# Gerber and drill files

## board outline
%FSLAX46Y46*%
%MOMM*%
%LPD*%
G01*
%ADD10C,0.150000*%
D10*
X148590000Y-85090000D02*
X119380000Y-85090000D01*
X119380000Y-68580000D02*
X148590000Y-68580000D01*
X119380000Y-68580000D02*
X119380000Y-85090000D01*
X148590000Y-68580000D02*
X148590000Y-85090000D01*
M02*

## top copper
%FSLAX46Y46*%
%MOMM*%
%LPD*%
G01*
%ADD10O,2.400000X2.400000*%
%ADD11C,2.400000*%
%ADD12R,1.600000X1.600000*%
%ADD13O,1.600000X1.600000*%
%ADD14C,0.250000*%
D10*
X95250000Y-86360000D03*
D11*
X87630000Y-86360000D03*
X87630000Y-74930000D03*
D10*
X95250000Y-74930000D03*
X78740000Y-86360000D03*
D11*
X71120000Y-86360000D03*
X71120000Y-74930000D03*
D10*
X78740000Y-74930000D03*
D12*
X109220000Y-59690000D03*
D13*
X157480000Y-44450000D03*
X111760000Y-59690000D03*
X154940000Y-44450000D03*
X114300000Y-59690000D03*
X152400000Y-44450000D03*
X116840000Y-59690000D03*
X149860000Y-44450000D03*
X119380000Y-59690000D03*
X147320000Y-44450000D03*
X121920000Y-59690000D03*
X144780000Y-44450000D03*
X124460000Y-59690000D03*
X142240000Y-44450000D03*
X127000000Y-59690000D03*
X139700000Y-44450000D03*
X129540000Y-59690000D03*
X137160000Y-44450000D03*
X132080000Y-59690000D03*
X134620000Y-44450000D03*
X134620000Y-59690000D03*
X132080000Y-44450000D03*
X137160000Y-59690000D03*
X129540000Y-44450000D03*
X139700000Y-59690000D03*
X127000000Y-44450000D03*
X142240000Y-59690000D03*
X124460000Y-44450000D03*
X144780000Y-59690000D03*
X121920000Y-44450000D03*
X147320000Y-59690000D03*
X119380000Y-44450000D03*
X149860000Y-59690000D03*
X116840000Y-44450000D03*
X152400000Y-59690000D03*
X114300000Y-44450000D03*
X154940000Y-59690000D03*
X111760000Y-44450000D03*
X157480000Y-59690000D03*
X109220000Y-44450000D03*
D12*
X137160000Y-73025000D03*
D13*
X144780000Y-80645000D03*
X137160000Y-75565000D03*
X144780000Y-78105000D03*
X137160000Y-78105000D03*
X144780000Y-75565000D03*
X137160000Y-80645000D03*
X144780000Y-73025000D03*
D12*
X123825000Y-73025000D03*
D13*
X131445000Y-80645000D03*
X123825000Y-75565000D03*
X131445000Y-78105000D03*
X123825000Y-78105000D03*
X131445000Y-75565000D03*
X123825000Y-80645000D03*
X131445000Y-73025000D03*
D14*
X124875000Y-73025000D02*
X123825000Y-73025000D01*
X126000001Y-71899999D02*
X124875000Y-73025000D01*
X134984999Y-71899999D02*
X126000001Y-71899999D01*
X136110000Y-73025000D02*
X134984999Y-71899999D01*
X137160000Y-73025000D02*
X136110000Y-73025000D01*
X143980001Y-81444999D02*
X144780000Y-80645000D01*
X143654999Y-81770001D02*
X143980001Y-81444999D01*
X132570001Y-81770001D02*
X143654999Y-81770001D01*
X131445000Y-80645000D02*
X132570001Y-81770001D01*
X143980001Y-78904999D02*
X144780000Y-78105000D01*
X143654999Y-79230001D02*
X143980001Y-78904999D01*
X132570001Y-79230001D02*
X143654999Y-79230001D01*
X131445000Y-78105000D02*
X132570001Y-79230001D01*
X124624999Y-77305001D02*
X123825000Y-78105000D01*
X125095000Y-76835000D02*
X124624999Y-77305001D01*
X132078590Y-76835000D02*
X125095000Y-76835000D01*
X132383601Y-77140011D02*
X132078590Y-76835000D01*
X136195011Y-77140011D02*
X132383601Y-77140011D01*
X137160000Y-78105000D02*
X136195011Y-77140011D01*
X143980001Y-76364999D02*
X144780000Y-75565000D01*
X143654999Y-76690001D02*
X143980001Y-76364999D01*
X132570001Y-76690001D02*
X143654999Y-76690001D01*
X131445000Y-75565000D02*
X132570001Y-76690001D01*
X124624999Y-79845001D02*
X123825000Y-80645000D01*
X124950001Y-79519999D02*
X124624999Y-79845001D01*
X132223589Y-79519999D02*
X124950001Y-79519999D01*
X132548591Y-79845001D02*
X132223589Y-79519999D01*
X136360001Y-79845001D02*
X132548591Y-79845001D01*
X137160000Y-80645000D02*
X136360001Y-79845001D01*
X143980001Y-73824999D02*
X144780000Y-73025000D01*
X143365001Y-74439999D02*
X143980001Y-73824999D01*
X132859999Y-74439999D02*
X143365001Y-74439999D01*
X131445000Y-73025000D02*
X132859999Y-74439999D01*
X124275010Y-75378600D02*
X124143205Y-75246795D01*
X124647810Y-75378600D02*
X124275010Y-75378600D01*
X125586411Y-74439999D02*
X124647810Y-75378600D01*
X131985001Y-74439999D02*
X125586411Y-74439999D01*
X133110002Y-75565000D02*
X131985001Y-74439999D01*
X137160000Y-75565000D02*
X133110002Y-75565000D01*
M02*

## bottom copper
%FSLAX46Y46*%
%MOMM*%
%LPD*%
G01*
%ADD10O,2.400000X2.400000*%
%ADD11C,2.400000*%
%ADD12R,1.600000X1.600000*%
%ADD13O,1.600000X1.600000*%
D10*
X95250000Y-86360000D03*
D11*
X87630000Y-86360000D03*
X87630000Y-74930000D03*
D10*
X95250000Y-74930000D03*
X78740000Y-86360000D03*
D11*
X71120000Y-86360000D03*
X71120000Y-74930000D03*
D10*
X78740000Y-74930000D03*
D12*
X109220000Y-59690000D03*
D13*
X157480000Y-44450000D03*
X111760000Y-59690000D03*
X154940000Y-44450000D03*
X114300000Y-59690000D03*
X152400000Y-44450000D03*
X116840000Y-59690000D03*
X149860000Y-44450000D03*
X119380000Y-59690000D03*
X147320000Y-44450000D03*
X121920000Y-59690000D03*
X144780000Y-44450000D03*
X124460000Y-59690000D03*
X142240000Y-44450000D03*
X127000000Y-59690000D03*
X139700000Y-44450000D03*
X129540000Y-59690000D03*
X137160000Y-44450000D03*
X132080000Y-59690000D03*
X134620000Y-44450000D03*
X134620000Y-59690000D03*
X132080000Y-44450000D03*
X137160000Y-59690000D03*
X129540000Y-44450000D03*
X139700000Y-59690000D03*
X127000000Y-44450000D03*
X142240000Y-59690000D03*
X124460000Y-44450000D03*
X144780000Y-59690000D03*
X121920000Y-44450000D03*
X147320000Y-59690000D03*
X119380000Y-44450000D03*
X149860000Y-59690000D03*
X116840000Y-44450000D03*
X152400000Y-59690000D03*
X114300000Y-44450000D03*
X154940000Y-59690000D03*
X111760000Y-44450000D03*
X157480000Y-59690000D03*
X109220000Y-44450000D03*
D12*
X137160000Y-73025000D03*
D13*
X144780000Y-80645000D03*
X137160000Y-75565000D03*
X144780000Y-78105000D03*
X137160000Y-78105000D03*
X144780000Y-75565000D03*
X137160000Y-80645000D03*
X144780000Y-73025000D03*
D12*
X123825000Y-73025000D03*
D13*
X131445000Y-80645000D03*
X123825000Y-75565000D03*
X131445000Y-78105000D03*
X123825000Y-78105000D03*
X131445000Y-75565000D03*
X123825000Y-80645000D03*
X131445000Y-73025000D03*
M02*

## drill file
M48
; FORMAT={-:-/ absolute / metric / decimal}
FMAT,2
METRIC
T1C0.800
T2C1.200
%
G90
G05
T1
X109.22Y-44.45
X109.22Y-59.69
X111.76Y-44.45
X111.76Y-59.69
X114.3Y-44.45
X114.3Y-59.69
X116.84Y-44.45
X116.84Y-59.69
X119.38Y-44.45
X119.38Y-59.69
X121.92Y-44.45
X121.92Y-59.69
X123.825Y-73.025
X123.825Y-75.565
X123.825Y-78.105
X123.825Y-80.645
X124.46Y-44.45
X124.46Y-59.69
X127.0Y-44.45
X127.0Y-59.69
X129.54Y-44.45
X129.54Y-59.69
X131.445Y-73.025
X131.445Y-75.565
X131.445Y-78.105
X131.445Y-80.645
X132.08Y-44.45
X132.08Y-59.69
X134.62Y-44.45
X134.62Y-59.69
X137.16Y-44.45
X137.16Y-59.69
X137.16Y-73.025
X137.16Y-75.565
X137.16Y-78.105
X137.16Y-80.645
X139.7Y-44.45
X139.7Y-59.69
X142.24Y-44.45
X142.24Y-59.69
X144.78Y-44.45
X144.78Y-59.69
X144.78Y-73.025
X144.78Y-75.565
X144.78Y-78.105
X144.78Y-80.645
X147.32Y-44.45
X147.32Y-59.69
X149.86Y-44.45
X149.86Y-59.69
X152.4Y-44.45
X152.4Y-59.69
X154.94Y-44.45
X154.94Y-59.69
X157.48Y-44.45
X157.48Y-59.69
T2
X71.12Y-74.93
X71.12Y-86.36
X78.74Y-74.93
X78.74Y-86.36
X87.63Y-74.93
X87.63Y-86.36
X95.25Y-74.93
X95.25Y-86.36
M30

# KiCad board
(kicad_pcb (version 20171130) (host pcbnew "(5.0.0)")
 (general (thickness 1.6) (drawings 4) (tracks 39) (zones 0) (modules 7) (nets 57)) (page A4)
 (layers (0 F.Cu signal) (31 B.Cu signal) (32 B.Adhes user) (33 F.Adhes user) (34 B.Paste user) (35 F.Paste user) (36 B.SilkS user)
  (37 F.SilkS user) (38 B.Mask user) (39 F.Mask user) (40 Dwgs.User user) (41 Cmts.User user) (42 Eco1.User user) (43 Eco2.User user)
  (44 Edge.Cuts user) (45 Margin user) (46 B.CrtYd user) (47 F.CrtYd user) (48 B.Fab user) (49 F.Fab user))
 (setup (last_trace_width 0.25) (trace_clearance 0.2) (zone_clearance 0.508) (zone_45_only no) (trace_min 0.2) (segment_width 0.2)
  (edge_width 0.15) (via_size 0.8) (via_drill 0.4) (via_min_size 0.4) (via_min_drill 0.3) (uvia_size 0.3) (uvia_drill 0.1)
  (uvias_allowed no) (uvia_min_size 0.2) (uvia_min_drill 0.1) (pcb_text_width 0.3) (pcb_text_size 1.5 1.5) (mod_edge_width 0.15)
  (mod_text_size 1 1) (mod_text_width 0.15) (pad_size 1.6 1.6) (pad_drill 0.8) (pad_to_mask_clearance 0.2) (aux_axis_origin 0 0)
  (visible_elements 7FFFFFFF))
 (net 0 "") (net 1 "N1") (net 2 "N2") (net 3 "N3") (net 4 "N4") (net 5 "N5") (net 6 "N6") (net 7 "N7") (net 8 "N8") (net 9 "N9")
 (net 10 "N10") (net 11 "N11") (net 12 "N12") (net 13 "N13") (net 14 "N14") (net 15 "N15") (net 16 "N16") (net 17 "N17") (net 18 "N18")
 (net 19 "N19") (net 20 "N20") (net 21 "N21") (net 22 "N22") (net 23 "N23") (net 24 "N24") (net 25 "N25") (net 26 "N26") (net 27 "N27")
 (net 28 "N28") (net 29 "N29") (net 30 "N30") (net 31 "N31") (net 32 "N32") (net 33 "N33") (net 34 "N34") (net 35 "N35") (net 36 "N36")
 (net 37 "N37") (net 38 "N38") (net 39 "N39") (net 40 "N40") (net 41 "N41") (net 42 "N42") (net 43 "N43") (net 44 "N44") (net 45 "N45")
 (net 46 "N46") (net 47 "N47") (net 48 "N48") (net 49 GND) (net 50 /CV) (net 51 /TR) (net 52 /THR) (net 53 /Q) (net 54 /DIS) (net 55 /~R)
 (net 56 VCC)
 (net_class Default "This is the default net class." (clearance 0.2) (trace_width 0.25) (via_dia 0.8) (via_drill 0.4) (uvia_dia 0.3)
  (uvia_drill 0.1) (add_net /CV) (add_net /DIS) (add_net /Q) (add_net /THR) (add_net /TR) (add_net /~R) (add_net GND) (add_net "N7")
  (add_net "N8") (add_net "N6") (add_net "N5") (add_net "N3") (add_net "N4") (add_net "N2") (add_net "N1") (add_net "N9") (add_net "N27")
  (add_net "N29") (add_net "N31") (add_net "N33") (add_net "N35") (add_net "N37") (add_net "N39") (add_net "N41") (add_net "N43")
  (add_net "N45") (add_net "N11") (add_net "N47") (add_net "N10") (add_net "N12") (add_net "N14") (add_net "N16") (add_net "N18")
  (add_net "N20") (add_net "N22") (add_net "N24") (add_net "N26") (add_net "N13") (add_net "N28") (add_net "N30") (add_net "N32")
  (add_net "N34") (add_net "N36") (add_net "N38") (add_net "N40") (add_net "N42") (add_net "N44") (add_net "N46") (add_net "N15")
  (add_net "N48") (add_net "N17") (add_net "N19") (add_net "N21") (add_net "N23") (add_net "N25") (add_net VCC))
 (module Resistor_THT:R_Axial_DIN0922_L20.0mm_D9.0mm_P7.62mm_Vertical (layer F.Cu) (at 87.63 86.36)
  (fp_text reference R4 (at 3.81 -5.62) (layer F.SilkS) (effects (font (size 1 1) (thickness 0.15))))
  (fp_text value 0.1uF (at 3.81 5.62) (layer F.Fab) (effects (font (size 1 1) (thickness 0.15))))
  (pad 2 thru_hole oval (at 7.62 0) (size 2.4 2.4) (drill 1.2) (layers *.Cu *.Mask) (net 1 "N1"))
  (pad 1 thru_hole circle (at 0 0) (size 2.4 2.4) (drill 1.2) (layers *.Cu *.Mask) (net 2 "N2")))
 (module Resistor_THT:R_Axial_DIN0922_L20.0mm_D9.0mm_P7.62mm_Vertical (layer F.Cu) (at 87.63 74.93)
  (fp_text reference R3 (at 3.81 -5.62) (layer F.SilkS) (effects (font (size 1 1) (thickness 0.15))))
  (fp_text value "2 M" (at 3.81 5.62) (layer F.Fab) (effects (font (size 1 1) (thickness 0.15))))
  (pad 1 thru_hole circle (at 0 0) (size 2.4 2.4) (drill 1.2) (layers *.Cu *.Mask) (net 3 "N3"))
  (pad 2 thru_hole oval (at 7.62 0) (size 2.4 2.4) (drill 1.2) (layers *.Cu *.Mask) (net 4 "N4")))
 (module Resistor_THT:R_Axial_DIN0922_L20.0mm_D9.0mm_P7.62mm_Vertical (layer F.Cu) (at 71.12 86.36)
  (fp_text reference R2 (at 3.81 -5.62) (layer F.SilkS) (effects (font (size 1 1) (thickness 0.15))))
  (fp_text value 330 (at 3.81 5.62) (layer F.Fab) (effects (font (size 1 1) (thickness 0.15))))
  (pad 2 thru_hole oval (at 7.62 0) (size 2.4 2.4) (drill 1.2) (layers *.Cu *.Mask) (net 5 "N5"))
  (pad 1 thru_hole circle (at 0 0) (size 2.4 2.4) (drill 1.2) (layers *.Cu *.Mask) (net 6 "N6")))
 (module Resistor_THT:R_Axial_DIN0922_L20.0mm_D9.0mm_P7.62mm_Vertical (layer F.Cu) (at 71.12 74.93)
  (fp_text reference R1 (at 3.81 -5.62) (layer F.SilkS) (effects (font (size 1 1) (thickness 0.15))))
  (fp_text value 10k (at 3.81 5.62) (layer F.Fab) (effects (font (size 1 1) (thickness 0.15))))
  (pad 1 thru_hole circle (at 0 0) (size 2.4 2.4) (drill 1.2) (layers *.Cu *.Mask) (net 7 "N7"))
  (pad 2 thru_hole oval (at 7.62 0) (size 2.4 2.4) (drill 1.2) (layers *.Cu *.Mask) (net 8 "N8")))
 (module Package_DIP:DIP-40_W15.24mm (layer F.Cu) (at 109.22 59.69 90)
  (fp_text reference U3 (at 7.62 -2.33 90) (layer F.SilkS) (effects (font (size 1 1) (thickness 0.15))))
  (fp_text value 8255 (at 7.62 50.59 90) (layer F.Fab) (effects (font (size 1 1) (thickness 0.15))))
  (pad 1 thru_hole rect (at 0 0 90) (size 1.6 1.6) (drill 0.8) (layers *.Cu *.Mask) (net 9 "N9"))
  (pad 21 thru_hole oval (at 15.24 48.26 90) (size 1.6 1.6) (drill 0.8) (layers *.Cu *.Mask) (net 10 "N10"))
  (pad 2 thru_hole oval (at 0 2.54 90) (size 1.6 1.6) (drill 0.8) (layers *.Cu *.Mask) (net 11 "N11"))
  (pad 22 thru_hole oval (at 15.24 45.72 90) (size 1.6 1.6) (drill 0.8) (layers *.Cu *.Mask) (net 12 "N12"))
  (pad 3 thru_hole oval (at 0 5.08 90) (size 1.6 1.6) (drill 0.8) (layers *.Cu *.Mask) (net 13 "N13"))
  (pad 23 thru_hole oval (at 15.24 43.18 90) (size 1.6 1.6) (drill 0.8) (layers *.Cu *.Mask) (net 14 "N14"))
  (pad 4 thru_hole oval (at 0 7.62 90) (size 1.6 1.6) (drill 0.8) (layers *.Cu *.Mask) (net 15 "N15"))
  (pad 24 thru_hole oval (at 15.24 40.64 90) (size 1.6 1.6) (drill 0.8) (layers *.Cu *.Mask) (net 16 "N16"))
  (pad 5 thru_hole oval (at 0 10.16 90) (size 1.6 1.6) (drill 0.8) (layers *.Cu *.Mask) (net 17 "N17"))
  (pad 25 thru_hole oval (at 15.24 38.1 90) (size 1.6 1.6) (drill 0.8) (layers *.Cu *.Mask) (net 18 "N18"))
  (pad 6 thru_hole oval (at 0 12.7 90) (size 1.6 1.6) (drill 0.8) (layers *.Cu *.Mask) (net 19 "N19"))
  (pad 26 thru_hole oval (at 15.24 35.56 90) (size 1.6 1.6) (drill 0.8) (layers *.Cu *.Mask) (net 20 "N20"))
  (pad 7 thru_hole oval (at 0 15.24 90) (size 1.6 1.6) (drill 0.8) (layers *.Cu *.Mask) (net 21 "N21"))
  (pad 27 thru_hole oval (at 15.24 33.02 90) (size 1.6 1.6) (drill 0.8) (layers *.Cu *.Mask) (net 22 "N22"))
  (pad 8 thru_hole oval (at 0 17.78 90) (size 1.6 1.6) (drill 0.8) (layers *.Cu *.Mask) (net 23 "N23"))
  (pad 28 thru_hole oval (at 15.24 30.48 90) (size 1.6 1.6) (drill 0.8) (layers *.Cu *.Mask) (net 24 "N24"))
  (pad 9 thru_hole oval (at 0 20.32 90) (size 1.6 1.6) (drill 0.8) (layers *.Cu *.Mask) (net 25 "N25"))
  (pad 29 thru_hole oval (at 15.24 27.94 90) (size 1.6 1.6) (drill 0.8) (layers *.Cu *.Mask) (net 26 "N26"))
  (pad 10 thru_hole oval (at 0 22.86 90) (size 1.6 1.6) (drill 0.8) (layers *.Cu *.Mask) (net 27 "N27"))
  (pad 30 thru_hole oval (at 15.24 25.4 90) (size 1.6 1.6) (drill 0.8) (layers *.Cu *.Mask) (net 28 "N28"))
  (pad 11 thru_hole oval (at 0 25.4 90) (size 1.6 1.6) (drill 0.8) (layers *.Cu *.Mask) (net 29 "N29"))
  (pad 31 thru_hole oval (at 15.24 22.86 90) (size 1.6 1.6) (drill 0.8) (layers *.Cu *.Mask) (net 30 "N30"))
  (pad 12 thru_hole oval (at 0 27.94 90) (size 1.6 1.6) (drill 0.8) (layers *.Cu *.Mask) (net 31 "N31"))
  (pad 32 thru_hole oval (at 15.24 20.32 90) (size 1.6 1.6) (drill 0.8) (layers *.Cu *.Mask) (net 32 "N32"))
  (pad 13 thru_hole oval (at 0 30.48 90) (size 1.6 1.6) (drill 0.8) (layers *.Cu *.Mask) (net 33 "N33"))
  (pad 33 thru_hole oval (at 15.24 17.78 90) (size 1.6 1.6) (drill 0.8) (layers *.Cu *.Mask) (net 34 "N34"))
  (pad 14 thru_hole oval (at 0 33.02 90) (size 1.6 1.6) (drill 0.8) (layers *.Cu *.Mask) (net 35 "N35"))
  (pad 34 thru_hole oval (at 15.24 15.24 90) (size 1.6 1.6) (drill 0.8) (layers *.Cu *.Mask) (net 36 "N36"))
  (pad 15 thru_hole oval (at 0 35.56 90) (size 1.6 1.6) (drill 0.8) (layers *.Cu *.Mask) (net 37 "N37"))
  (pad 35 thru_hole oval (at 15.24 12.7 90) (size 1.6 1.6) (drill 0.8) (layers *.Cu *.Mask) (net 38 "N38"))
  (pad 16 thru_hole oval (at 0 38.1 90) (size 1.6 1.6) (drill 0.8) (layers *.Cu *.Mask) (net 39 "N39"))
  (pad 36 thru_hole oval (at 15.24 10.16 90) (size 1.6 1.6) (drill 0.8) (layers *.Cu *.Mask) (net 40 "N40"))
  (pad 17 thru_hole oval (at 0 40.64 90) (size 1.6 1.6) (drill 0.8) (layers *.Cu *.Mask) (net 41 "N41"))
  (pad 37 thru_hole oval (at 15.24 7.62 90) (size 1.6 1.6) (drill 0.8) (layers *.Cu *.Mask) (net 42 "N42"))
  (pad 18 thru_hole oval (at 0 43.18 90) (size 1.6 1.6) (drill 0.8) (layers *.Cu *.Mask) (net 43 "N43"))
  (pad 38 thru_hole oval (at 15.24 5.08 90) (size 1.6 1.6) (drill 0.8) (layers *.Cu *.Mask) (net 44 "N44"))
  (pad 19 thru_hole oval (at 0 45.72 90) (size 1.6 1.6) (drill 0.8) (layers *.Cu *.Mask) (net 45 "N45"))
  (pad 39 thru_hole oval (at 15.24 2.54 90) (size 1.6 1.6) (drill 0.8) (layers *.Cu *.Mask) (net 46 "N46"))
  (pad 20 thru_hole oval (at 0 48.26 90) (size 1.6 1.6) (drill 0.8) (layers *.Cu *.Mask) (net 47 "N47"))
  (pad 40 thru_hole oval (at 15.24 0 90) (size 1.6 1.6) (drill 0.8) (layers *.Cu *.Mask) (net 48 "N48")))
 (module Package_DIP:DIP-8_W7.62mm (layer F.Cu) (at 137.16 73.025)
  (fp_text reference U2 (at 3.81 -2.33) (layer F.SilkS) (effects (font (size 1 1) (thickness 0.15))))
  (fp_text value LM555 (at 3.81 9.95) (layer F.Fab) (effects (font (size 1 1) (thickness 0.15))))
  (pad 1 thru_hole rect (at 0 0) (size 1.6 1.6) (drill 0.8) (layers *.Cu *.Mask) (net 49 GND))
  (pad 5 thru_hole oval (at 7.62 7.62) (size 1.6 1.6) (drill 0.8) (layers *.Cu *.Mask) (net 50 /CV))
  (pad 2 thru_hole oval (at 0 2.54) (size 1.6 1.6) (drill 0.8) (layers *.Cu *.Mask) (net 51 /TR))
  (pad 6 thru_hole oval (at 7.62 5.08) (size 1.6 1.6) (drill 0.8) (layers *.Cu *.Mask) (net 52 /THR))
  (pad 3 thru_hole oval (at 0 5.08) (size 1.6 1.6) (drill 0.8) (layers *.Cu *.Mask) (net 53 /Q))
  (pad 7 thru_hole oval (at 7.62 2.54) (size 1.6 1.6) (drill 0.8) (layers *.Cu *.Mask) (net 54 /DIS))
  (pad 4 thru_hole oval (at 0 7.62) (size 1.6 1.6) (drill 0.8) (layers *.Cu *.Mask) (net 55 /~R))
  (pad 8 thru_hole oval (at 7.62 0) (size 1.6 1.6) (drill 0.8) (layers *.Cu *.Mask) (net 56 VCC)))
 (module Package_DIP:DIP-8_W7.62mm (layer F.Cu) (at 123.825 73.025)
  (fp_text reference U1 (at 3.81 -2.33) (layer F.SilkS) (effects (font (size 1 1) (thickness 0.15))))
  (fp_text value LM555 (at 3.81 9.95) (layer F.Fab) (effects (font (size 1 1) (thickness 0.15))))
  (pad 1 thru_hole rect (at 0 0) (size 1.6 1.6) (drill 0.8) (layers *.Cu *.Mask) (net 49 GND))
  (pad 5 thru_hole oval (at 7.62 7.62) (size 1.6 1.6) (drill 0.8) (layers *.Cu *.Mask) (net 50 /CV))
  (pad 2 thru_hole oval (at 0 2.54) (size 1.6 1.6) (drill 0.8) (layers *.Cu *.Mask) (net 51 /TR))
  (pad 6 thru_hole oval (at 7.62 5.08) (size 1.6 1.6) (drill 0.8) (layers *.Cu *.Mask) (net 52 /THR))
  (pad 3 thru_hole oval (at 0 5.08) (size 1.6 1.6) (drill 0.8) (layers *.Cu *.Mask) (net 53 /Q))
  (pad 7 thru_hole oval (at 7.62 2.54) (size 1.6 1.6) (drill 0.8) (layers *.Cu *.Mask) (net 54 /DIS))
  (pad 4 thru_hole oval (at 0 7.62) (size 1.6 1.6) (drill 0.8) (layers *.Cu *.Mask) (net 55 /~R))
  (pad 8 thru_hole oval (at 7.62 0) (size 1.6 1.6) (drill 0.8) (layers *.Cu *.Mask) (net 56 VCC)))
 (gr_line (start 148.59 85.09) (end 119.38 85.09) (layer Edge.Cuts) (width 0.15))
 (gr_line (start 119.38 68.58) (end 148.59 68.58) (layer Edge.Cuts) (width 0.15))
 (gr_line (start 119.38 68.58) (end 119.38 85.09) (layer Edge.Cuts) (width 0.15))
 (gr_line (start 148.59 68.58) (end 148.59 85.09) (layer Edge.Cuts) (width 0.15))
 (segment (start 124.875 73.025) (end 123.825 73.025) (width 0.25) (layer F.Cu) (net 49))
 (segment (start 126.000001 71.899999) (end 124.875 73.025) (width 0.25) (layer F.Cu) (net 49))
 (segment (start 134.984999 71.899999) (end 126.000001 71.899999) (width 0.25) (layer F.Cu) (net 49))
 (segment (start 136.11 73.025) (end 134.984999 71.899999) (width 0.25) (layer F.Cu) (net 49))
 (segment (start 137.16 73.025) (end 136.11 73.025) (width 0.25) (layer F.Cu) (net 49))
 (segment (start 143.980001 81.444999) (end 144.78 80.645) (width 0.25) (layer F.Cu) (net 50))
 (segment (start 143.654999 81.770001) (end 143.980001 81.444999) (width 0.25) (layer F.Cu) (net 50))
 (segment (start 132.570001 81.770001) (end 143.654999 81.770001) (width 0.25) (layer F.Cu) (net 50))
 (segment (start 131.445 80.645) (end 132.570001 81.770001) (width 0.25) (layer F.Cu) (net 50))
 (segment (start 143.980001 78.904999) (end 144.78 78.105) (width 0.25) (layer F.Cu) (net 52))
 (segment (start 143.654999 79.230001) (end 143.980001 78.904999) (width 0.25) (layer F.Cu) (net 52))
 (segment (start 132.570001 79.230001) (end 143.654999 79.230001) (width 0.25) (layer F.Cu) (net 52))
 (segment (start 131.445 78.105) (end 132.570001 79.230001) (width 0.25) (layer F.Cu) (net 52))
 (segment (start 124.624999 77.305001) (end 123.825 78.105) (width 0.25) (layer F.Cu) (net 53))
 (segment (start 125.095 76.835) (end 124.624999 77.305001) (width 0.25) (layer F.Cu) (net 53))
 (segment (start 132.07859 76.835) (end 125.095 76.835) (width 0.25) (layer F.Cu) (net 53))
 (segment (start 132.383601 77.140011) (end 132.07859 76.835) (width 0.25) (layer F.Cu) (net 53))
 (segment (start 136.195011 77.140011) (end 132.383601 77.140011) (width 0.25) (layer F.Cu) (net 53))
 (segment (start 137.16 78.105) (end 136.195011 77.140011) (width 0.25) (layer F.Cu) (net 53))
 (segment (start 143.980001 76.364999) (end 144.78 75.565) (width 0.25) (layer F.Cu) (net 54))
 (segment (start 143.654999 76.690001) (end 143.980001 76.364999) (width 0.25) (layer F.Cu) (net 54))
 (segment (start 132.570001 76.690001) (end 143.654999 76.690001) (width 0.25) (layer F.Cu) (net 54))
 (segment (start 131.445 75.565) (end 132.570001 76.690001) (width 0.25) (layer F.Cu) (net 54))
 (segment (start 124.624999 79.845001) (end 123.825 80.645) (width 0.25) (layer F.Cu) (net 55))
 (segment (start 124.950001 79.519999) (end 124.624999 79.845001) (width 0.25) (layer F.Cu) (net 55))
 (segment (start 132.223589 79.519999) (end 124.950001 79.519999) (width 0.25) (layer F.Cu) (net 55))
 (segment (start 132.548591 79.845001) (end 132.223589 79.519999) (width 0.25) (layer F.Cu) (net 55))
 (segment (start 136.360001 79.845001) (end 132.548591 79.845001) (width 0.25) (layer F.Cu) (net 55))
 (segment (start 137.16 80.645) (end 136.360001 79.845001) (width 0.25) (layer F.Cu) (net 55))
 (segment (start 143.980001 73.824999) (end 144.78 73.025) (width 0.25) (layer F.Cu) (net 56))
 (segment (start 143.365001 74.439999) (end 143.980001 73.824999) (width 0.25) (layer F.Cu) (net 56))
 (segment (start 132.859999 74.439999) (end 143.365001 74.439999) (width 0.25) (layer F.Cu) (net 56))
 (segment (start 131.445 73.025) (end 132.859999 74.439999) (width 0.25) (layer F.Cu) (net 56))
 (segment (start 124.27501 75.3786) (end 124.143205 75.246795) (width 0.25) (layer F.Cu) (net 51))
 (segment (start 124.64781 75.3786) (end 124.27501 75.3786) (width 0.25) (layer F.Cu) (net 51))
 (segment (start 125.586411 74.439999) (end 124.64781 75.3786) (width 0.25) (layer F.Cu) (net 51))
 (segment (start 131.985001 74.439999) (end 125.586411 74.439999) (width 0.25) (layer F.Cu) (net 51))
 (segment (start 133.110002 75.565) (end 131.985001 74.439999) (width 0.25) (layer F.Cu) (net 51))
 (segment (start 137.16 75.565) (end 133.110002 75.565) (width 0.25) (layer F.Cu) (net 51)))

